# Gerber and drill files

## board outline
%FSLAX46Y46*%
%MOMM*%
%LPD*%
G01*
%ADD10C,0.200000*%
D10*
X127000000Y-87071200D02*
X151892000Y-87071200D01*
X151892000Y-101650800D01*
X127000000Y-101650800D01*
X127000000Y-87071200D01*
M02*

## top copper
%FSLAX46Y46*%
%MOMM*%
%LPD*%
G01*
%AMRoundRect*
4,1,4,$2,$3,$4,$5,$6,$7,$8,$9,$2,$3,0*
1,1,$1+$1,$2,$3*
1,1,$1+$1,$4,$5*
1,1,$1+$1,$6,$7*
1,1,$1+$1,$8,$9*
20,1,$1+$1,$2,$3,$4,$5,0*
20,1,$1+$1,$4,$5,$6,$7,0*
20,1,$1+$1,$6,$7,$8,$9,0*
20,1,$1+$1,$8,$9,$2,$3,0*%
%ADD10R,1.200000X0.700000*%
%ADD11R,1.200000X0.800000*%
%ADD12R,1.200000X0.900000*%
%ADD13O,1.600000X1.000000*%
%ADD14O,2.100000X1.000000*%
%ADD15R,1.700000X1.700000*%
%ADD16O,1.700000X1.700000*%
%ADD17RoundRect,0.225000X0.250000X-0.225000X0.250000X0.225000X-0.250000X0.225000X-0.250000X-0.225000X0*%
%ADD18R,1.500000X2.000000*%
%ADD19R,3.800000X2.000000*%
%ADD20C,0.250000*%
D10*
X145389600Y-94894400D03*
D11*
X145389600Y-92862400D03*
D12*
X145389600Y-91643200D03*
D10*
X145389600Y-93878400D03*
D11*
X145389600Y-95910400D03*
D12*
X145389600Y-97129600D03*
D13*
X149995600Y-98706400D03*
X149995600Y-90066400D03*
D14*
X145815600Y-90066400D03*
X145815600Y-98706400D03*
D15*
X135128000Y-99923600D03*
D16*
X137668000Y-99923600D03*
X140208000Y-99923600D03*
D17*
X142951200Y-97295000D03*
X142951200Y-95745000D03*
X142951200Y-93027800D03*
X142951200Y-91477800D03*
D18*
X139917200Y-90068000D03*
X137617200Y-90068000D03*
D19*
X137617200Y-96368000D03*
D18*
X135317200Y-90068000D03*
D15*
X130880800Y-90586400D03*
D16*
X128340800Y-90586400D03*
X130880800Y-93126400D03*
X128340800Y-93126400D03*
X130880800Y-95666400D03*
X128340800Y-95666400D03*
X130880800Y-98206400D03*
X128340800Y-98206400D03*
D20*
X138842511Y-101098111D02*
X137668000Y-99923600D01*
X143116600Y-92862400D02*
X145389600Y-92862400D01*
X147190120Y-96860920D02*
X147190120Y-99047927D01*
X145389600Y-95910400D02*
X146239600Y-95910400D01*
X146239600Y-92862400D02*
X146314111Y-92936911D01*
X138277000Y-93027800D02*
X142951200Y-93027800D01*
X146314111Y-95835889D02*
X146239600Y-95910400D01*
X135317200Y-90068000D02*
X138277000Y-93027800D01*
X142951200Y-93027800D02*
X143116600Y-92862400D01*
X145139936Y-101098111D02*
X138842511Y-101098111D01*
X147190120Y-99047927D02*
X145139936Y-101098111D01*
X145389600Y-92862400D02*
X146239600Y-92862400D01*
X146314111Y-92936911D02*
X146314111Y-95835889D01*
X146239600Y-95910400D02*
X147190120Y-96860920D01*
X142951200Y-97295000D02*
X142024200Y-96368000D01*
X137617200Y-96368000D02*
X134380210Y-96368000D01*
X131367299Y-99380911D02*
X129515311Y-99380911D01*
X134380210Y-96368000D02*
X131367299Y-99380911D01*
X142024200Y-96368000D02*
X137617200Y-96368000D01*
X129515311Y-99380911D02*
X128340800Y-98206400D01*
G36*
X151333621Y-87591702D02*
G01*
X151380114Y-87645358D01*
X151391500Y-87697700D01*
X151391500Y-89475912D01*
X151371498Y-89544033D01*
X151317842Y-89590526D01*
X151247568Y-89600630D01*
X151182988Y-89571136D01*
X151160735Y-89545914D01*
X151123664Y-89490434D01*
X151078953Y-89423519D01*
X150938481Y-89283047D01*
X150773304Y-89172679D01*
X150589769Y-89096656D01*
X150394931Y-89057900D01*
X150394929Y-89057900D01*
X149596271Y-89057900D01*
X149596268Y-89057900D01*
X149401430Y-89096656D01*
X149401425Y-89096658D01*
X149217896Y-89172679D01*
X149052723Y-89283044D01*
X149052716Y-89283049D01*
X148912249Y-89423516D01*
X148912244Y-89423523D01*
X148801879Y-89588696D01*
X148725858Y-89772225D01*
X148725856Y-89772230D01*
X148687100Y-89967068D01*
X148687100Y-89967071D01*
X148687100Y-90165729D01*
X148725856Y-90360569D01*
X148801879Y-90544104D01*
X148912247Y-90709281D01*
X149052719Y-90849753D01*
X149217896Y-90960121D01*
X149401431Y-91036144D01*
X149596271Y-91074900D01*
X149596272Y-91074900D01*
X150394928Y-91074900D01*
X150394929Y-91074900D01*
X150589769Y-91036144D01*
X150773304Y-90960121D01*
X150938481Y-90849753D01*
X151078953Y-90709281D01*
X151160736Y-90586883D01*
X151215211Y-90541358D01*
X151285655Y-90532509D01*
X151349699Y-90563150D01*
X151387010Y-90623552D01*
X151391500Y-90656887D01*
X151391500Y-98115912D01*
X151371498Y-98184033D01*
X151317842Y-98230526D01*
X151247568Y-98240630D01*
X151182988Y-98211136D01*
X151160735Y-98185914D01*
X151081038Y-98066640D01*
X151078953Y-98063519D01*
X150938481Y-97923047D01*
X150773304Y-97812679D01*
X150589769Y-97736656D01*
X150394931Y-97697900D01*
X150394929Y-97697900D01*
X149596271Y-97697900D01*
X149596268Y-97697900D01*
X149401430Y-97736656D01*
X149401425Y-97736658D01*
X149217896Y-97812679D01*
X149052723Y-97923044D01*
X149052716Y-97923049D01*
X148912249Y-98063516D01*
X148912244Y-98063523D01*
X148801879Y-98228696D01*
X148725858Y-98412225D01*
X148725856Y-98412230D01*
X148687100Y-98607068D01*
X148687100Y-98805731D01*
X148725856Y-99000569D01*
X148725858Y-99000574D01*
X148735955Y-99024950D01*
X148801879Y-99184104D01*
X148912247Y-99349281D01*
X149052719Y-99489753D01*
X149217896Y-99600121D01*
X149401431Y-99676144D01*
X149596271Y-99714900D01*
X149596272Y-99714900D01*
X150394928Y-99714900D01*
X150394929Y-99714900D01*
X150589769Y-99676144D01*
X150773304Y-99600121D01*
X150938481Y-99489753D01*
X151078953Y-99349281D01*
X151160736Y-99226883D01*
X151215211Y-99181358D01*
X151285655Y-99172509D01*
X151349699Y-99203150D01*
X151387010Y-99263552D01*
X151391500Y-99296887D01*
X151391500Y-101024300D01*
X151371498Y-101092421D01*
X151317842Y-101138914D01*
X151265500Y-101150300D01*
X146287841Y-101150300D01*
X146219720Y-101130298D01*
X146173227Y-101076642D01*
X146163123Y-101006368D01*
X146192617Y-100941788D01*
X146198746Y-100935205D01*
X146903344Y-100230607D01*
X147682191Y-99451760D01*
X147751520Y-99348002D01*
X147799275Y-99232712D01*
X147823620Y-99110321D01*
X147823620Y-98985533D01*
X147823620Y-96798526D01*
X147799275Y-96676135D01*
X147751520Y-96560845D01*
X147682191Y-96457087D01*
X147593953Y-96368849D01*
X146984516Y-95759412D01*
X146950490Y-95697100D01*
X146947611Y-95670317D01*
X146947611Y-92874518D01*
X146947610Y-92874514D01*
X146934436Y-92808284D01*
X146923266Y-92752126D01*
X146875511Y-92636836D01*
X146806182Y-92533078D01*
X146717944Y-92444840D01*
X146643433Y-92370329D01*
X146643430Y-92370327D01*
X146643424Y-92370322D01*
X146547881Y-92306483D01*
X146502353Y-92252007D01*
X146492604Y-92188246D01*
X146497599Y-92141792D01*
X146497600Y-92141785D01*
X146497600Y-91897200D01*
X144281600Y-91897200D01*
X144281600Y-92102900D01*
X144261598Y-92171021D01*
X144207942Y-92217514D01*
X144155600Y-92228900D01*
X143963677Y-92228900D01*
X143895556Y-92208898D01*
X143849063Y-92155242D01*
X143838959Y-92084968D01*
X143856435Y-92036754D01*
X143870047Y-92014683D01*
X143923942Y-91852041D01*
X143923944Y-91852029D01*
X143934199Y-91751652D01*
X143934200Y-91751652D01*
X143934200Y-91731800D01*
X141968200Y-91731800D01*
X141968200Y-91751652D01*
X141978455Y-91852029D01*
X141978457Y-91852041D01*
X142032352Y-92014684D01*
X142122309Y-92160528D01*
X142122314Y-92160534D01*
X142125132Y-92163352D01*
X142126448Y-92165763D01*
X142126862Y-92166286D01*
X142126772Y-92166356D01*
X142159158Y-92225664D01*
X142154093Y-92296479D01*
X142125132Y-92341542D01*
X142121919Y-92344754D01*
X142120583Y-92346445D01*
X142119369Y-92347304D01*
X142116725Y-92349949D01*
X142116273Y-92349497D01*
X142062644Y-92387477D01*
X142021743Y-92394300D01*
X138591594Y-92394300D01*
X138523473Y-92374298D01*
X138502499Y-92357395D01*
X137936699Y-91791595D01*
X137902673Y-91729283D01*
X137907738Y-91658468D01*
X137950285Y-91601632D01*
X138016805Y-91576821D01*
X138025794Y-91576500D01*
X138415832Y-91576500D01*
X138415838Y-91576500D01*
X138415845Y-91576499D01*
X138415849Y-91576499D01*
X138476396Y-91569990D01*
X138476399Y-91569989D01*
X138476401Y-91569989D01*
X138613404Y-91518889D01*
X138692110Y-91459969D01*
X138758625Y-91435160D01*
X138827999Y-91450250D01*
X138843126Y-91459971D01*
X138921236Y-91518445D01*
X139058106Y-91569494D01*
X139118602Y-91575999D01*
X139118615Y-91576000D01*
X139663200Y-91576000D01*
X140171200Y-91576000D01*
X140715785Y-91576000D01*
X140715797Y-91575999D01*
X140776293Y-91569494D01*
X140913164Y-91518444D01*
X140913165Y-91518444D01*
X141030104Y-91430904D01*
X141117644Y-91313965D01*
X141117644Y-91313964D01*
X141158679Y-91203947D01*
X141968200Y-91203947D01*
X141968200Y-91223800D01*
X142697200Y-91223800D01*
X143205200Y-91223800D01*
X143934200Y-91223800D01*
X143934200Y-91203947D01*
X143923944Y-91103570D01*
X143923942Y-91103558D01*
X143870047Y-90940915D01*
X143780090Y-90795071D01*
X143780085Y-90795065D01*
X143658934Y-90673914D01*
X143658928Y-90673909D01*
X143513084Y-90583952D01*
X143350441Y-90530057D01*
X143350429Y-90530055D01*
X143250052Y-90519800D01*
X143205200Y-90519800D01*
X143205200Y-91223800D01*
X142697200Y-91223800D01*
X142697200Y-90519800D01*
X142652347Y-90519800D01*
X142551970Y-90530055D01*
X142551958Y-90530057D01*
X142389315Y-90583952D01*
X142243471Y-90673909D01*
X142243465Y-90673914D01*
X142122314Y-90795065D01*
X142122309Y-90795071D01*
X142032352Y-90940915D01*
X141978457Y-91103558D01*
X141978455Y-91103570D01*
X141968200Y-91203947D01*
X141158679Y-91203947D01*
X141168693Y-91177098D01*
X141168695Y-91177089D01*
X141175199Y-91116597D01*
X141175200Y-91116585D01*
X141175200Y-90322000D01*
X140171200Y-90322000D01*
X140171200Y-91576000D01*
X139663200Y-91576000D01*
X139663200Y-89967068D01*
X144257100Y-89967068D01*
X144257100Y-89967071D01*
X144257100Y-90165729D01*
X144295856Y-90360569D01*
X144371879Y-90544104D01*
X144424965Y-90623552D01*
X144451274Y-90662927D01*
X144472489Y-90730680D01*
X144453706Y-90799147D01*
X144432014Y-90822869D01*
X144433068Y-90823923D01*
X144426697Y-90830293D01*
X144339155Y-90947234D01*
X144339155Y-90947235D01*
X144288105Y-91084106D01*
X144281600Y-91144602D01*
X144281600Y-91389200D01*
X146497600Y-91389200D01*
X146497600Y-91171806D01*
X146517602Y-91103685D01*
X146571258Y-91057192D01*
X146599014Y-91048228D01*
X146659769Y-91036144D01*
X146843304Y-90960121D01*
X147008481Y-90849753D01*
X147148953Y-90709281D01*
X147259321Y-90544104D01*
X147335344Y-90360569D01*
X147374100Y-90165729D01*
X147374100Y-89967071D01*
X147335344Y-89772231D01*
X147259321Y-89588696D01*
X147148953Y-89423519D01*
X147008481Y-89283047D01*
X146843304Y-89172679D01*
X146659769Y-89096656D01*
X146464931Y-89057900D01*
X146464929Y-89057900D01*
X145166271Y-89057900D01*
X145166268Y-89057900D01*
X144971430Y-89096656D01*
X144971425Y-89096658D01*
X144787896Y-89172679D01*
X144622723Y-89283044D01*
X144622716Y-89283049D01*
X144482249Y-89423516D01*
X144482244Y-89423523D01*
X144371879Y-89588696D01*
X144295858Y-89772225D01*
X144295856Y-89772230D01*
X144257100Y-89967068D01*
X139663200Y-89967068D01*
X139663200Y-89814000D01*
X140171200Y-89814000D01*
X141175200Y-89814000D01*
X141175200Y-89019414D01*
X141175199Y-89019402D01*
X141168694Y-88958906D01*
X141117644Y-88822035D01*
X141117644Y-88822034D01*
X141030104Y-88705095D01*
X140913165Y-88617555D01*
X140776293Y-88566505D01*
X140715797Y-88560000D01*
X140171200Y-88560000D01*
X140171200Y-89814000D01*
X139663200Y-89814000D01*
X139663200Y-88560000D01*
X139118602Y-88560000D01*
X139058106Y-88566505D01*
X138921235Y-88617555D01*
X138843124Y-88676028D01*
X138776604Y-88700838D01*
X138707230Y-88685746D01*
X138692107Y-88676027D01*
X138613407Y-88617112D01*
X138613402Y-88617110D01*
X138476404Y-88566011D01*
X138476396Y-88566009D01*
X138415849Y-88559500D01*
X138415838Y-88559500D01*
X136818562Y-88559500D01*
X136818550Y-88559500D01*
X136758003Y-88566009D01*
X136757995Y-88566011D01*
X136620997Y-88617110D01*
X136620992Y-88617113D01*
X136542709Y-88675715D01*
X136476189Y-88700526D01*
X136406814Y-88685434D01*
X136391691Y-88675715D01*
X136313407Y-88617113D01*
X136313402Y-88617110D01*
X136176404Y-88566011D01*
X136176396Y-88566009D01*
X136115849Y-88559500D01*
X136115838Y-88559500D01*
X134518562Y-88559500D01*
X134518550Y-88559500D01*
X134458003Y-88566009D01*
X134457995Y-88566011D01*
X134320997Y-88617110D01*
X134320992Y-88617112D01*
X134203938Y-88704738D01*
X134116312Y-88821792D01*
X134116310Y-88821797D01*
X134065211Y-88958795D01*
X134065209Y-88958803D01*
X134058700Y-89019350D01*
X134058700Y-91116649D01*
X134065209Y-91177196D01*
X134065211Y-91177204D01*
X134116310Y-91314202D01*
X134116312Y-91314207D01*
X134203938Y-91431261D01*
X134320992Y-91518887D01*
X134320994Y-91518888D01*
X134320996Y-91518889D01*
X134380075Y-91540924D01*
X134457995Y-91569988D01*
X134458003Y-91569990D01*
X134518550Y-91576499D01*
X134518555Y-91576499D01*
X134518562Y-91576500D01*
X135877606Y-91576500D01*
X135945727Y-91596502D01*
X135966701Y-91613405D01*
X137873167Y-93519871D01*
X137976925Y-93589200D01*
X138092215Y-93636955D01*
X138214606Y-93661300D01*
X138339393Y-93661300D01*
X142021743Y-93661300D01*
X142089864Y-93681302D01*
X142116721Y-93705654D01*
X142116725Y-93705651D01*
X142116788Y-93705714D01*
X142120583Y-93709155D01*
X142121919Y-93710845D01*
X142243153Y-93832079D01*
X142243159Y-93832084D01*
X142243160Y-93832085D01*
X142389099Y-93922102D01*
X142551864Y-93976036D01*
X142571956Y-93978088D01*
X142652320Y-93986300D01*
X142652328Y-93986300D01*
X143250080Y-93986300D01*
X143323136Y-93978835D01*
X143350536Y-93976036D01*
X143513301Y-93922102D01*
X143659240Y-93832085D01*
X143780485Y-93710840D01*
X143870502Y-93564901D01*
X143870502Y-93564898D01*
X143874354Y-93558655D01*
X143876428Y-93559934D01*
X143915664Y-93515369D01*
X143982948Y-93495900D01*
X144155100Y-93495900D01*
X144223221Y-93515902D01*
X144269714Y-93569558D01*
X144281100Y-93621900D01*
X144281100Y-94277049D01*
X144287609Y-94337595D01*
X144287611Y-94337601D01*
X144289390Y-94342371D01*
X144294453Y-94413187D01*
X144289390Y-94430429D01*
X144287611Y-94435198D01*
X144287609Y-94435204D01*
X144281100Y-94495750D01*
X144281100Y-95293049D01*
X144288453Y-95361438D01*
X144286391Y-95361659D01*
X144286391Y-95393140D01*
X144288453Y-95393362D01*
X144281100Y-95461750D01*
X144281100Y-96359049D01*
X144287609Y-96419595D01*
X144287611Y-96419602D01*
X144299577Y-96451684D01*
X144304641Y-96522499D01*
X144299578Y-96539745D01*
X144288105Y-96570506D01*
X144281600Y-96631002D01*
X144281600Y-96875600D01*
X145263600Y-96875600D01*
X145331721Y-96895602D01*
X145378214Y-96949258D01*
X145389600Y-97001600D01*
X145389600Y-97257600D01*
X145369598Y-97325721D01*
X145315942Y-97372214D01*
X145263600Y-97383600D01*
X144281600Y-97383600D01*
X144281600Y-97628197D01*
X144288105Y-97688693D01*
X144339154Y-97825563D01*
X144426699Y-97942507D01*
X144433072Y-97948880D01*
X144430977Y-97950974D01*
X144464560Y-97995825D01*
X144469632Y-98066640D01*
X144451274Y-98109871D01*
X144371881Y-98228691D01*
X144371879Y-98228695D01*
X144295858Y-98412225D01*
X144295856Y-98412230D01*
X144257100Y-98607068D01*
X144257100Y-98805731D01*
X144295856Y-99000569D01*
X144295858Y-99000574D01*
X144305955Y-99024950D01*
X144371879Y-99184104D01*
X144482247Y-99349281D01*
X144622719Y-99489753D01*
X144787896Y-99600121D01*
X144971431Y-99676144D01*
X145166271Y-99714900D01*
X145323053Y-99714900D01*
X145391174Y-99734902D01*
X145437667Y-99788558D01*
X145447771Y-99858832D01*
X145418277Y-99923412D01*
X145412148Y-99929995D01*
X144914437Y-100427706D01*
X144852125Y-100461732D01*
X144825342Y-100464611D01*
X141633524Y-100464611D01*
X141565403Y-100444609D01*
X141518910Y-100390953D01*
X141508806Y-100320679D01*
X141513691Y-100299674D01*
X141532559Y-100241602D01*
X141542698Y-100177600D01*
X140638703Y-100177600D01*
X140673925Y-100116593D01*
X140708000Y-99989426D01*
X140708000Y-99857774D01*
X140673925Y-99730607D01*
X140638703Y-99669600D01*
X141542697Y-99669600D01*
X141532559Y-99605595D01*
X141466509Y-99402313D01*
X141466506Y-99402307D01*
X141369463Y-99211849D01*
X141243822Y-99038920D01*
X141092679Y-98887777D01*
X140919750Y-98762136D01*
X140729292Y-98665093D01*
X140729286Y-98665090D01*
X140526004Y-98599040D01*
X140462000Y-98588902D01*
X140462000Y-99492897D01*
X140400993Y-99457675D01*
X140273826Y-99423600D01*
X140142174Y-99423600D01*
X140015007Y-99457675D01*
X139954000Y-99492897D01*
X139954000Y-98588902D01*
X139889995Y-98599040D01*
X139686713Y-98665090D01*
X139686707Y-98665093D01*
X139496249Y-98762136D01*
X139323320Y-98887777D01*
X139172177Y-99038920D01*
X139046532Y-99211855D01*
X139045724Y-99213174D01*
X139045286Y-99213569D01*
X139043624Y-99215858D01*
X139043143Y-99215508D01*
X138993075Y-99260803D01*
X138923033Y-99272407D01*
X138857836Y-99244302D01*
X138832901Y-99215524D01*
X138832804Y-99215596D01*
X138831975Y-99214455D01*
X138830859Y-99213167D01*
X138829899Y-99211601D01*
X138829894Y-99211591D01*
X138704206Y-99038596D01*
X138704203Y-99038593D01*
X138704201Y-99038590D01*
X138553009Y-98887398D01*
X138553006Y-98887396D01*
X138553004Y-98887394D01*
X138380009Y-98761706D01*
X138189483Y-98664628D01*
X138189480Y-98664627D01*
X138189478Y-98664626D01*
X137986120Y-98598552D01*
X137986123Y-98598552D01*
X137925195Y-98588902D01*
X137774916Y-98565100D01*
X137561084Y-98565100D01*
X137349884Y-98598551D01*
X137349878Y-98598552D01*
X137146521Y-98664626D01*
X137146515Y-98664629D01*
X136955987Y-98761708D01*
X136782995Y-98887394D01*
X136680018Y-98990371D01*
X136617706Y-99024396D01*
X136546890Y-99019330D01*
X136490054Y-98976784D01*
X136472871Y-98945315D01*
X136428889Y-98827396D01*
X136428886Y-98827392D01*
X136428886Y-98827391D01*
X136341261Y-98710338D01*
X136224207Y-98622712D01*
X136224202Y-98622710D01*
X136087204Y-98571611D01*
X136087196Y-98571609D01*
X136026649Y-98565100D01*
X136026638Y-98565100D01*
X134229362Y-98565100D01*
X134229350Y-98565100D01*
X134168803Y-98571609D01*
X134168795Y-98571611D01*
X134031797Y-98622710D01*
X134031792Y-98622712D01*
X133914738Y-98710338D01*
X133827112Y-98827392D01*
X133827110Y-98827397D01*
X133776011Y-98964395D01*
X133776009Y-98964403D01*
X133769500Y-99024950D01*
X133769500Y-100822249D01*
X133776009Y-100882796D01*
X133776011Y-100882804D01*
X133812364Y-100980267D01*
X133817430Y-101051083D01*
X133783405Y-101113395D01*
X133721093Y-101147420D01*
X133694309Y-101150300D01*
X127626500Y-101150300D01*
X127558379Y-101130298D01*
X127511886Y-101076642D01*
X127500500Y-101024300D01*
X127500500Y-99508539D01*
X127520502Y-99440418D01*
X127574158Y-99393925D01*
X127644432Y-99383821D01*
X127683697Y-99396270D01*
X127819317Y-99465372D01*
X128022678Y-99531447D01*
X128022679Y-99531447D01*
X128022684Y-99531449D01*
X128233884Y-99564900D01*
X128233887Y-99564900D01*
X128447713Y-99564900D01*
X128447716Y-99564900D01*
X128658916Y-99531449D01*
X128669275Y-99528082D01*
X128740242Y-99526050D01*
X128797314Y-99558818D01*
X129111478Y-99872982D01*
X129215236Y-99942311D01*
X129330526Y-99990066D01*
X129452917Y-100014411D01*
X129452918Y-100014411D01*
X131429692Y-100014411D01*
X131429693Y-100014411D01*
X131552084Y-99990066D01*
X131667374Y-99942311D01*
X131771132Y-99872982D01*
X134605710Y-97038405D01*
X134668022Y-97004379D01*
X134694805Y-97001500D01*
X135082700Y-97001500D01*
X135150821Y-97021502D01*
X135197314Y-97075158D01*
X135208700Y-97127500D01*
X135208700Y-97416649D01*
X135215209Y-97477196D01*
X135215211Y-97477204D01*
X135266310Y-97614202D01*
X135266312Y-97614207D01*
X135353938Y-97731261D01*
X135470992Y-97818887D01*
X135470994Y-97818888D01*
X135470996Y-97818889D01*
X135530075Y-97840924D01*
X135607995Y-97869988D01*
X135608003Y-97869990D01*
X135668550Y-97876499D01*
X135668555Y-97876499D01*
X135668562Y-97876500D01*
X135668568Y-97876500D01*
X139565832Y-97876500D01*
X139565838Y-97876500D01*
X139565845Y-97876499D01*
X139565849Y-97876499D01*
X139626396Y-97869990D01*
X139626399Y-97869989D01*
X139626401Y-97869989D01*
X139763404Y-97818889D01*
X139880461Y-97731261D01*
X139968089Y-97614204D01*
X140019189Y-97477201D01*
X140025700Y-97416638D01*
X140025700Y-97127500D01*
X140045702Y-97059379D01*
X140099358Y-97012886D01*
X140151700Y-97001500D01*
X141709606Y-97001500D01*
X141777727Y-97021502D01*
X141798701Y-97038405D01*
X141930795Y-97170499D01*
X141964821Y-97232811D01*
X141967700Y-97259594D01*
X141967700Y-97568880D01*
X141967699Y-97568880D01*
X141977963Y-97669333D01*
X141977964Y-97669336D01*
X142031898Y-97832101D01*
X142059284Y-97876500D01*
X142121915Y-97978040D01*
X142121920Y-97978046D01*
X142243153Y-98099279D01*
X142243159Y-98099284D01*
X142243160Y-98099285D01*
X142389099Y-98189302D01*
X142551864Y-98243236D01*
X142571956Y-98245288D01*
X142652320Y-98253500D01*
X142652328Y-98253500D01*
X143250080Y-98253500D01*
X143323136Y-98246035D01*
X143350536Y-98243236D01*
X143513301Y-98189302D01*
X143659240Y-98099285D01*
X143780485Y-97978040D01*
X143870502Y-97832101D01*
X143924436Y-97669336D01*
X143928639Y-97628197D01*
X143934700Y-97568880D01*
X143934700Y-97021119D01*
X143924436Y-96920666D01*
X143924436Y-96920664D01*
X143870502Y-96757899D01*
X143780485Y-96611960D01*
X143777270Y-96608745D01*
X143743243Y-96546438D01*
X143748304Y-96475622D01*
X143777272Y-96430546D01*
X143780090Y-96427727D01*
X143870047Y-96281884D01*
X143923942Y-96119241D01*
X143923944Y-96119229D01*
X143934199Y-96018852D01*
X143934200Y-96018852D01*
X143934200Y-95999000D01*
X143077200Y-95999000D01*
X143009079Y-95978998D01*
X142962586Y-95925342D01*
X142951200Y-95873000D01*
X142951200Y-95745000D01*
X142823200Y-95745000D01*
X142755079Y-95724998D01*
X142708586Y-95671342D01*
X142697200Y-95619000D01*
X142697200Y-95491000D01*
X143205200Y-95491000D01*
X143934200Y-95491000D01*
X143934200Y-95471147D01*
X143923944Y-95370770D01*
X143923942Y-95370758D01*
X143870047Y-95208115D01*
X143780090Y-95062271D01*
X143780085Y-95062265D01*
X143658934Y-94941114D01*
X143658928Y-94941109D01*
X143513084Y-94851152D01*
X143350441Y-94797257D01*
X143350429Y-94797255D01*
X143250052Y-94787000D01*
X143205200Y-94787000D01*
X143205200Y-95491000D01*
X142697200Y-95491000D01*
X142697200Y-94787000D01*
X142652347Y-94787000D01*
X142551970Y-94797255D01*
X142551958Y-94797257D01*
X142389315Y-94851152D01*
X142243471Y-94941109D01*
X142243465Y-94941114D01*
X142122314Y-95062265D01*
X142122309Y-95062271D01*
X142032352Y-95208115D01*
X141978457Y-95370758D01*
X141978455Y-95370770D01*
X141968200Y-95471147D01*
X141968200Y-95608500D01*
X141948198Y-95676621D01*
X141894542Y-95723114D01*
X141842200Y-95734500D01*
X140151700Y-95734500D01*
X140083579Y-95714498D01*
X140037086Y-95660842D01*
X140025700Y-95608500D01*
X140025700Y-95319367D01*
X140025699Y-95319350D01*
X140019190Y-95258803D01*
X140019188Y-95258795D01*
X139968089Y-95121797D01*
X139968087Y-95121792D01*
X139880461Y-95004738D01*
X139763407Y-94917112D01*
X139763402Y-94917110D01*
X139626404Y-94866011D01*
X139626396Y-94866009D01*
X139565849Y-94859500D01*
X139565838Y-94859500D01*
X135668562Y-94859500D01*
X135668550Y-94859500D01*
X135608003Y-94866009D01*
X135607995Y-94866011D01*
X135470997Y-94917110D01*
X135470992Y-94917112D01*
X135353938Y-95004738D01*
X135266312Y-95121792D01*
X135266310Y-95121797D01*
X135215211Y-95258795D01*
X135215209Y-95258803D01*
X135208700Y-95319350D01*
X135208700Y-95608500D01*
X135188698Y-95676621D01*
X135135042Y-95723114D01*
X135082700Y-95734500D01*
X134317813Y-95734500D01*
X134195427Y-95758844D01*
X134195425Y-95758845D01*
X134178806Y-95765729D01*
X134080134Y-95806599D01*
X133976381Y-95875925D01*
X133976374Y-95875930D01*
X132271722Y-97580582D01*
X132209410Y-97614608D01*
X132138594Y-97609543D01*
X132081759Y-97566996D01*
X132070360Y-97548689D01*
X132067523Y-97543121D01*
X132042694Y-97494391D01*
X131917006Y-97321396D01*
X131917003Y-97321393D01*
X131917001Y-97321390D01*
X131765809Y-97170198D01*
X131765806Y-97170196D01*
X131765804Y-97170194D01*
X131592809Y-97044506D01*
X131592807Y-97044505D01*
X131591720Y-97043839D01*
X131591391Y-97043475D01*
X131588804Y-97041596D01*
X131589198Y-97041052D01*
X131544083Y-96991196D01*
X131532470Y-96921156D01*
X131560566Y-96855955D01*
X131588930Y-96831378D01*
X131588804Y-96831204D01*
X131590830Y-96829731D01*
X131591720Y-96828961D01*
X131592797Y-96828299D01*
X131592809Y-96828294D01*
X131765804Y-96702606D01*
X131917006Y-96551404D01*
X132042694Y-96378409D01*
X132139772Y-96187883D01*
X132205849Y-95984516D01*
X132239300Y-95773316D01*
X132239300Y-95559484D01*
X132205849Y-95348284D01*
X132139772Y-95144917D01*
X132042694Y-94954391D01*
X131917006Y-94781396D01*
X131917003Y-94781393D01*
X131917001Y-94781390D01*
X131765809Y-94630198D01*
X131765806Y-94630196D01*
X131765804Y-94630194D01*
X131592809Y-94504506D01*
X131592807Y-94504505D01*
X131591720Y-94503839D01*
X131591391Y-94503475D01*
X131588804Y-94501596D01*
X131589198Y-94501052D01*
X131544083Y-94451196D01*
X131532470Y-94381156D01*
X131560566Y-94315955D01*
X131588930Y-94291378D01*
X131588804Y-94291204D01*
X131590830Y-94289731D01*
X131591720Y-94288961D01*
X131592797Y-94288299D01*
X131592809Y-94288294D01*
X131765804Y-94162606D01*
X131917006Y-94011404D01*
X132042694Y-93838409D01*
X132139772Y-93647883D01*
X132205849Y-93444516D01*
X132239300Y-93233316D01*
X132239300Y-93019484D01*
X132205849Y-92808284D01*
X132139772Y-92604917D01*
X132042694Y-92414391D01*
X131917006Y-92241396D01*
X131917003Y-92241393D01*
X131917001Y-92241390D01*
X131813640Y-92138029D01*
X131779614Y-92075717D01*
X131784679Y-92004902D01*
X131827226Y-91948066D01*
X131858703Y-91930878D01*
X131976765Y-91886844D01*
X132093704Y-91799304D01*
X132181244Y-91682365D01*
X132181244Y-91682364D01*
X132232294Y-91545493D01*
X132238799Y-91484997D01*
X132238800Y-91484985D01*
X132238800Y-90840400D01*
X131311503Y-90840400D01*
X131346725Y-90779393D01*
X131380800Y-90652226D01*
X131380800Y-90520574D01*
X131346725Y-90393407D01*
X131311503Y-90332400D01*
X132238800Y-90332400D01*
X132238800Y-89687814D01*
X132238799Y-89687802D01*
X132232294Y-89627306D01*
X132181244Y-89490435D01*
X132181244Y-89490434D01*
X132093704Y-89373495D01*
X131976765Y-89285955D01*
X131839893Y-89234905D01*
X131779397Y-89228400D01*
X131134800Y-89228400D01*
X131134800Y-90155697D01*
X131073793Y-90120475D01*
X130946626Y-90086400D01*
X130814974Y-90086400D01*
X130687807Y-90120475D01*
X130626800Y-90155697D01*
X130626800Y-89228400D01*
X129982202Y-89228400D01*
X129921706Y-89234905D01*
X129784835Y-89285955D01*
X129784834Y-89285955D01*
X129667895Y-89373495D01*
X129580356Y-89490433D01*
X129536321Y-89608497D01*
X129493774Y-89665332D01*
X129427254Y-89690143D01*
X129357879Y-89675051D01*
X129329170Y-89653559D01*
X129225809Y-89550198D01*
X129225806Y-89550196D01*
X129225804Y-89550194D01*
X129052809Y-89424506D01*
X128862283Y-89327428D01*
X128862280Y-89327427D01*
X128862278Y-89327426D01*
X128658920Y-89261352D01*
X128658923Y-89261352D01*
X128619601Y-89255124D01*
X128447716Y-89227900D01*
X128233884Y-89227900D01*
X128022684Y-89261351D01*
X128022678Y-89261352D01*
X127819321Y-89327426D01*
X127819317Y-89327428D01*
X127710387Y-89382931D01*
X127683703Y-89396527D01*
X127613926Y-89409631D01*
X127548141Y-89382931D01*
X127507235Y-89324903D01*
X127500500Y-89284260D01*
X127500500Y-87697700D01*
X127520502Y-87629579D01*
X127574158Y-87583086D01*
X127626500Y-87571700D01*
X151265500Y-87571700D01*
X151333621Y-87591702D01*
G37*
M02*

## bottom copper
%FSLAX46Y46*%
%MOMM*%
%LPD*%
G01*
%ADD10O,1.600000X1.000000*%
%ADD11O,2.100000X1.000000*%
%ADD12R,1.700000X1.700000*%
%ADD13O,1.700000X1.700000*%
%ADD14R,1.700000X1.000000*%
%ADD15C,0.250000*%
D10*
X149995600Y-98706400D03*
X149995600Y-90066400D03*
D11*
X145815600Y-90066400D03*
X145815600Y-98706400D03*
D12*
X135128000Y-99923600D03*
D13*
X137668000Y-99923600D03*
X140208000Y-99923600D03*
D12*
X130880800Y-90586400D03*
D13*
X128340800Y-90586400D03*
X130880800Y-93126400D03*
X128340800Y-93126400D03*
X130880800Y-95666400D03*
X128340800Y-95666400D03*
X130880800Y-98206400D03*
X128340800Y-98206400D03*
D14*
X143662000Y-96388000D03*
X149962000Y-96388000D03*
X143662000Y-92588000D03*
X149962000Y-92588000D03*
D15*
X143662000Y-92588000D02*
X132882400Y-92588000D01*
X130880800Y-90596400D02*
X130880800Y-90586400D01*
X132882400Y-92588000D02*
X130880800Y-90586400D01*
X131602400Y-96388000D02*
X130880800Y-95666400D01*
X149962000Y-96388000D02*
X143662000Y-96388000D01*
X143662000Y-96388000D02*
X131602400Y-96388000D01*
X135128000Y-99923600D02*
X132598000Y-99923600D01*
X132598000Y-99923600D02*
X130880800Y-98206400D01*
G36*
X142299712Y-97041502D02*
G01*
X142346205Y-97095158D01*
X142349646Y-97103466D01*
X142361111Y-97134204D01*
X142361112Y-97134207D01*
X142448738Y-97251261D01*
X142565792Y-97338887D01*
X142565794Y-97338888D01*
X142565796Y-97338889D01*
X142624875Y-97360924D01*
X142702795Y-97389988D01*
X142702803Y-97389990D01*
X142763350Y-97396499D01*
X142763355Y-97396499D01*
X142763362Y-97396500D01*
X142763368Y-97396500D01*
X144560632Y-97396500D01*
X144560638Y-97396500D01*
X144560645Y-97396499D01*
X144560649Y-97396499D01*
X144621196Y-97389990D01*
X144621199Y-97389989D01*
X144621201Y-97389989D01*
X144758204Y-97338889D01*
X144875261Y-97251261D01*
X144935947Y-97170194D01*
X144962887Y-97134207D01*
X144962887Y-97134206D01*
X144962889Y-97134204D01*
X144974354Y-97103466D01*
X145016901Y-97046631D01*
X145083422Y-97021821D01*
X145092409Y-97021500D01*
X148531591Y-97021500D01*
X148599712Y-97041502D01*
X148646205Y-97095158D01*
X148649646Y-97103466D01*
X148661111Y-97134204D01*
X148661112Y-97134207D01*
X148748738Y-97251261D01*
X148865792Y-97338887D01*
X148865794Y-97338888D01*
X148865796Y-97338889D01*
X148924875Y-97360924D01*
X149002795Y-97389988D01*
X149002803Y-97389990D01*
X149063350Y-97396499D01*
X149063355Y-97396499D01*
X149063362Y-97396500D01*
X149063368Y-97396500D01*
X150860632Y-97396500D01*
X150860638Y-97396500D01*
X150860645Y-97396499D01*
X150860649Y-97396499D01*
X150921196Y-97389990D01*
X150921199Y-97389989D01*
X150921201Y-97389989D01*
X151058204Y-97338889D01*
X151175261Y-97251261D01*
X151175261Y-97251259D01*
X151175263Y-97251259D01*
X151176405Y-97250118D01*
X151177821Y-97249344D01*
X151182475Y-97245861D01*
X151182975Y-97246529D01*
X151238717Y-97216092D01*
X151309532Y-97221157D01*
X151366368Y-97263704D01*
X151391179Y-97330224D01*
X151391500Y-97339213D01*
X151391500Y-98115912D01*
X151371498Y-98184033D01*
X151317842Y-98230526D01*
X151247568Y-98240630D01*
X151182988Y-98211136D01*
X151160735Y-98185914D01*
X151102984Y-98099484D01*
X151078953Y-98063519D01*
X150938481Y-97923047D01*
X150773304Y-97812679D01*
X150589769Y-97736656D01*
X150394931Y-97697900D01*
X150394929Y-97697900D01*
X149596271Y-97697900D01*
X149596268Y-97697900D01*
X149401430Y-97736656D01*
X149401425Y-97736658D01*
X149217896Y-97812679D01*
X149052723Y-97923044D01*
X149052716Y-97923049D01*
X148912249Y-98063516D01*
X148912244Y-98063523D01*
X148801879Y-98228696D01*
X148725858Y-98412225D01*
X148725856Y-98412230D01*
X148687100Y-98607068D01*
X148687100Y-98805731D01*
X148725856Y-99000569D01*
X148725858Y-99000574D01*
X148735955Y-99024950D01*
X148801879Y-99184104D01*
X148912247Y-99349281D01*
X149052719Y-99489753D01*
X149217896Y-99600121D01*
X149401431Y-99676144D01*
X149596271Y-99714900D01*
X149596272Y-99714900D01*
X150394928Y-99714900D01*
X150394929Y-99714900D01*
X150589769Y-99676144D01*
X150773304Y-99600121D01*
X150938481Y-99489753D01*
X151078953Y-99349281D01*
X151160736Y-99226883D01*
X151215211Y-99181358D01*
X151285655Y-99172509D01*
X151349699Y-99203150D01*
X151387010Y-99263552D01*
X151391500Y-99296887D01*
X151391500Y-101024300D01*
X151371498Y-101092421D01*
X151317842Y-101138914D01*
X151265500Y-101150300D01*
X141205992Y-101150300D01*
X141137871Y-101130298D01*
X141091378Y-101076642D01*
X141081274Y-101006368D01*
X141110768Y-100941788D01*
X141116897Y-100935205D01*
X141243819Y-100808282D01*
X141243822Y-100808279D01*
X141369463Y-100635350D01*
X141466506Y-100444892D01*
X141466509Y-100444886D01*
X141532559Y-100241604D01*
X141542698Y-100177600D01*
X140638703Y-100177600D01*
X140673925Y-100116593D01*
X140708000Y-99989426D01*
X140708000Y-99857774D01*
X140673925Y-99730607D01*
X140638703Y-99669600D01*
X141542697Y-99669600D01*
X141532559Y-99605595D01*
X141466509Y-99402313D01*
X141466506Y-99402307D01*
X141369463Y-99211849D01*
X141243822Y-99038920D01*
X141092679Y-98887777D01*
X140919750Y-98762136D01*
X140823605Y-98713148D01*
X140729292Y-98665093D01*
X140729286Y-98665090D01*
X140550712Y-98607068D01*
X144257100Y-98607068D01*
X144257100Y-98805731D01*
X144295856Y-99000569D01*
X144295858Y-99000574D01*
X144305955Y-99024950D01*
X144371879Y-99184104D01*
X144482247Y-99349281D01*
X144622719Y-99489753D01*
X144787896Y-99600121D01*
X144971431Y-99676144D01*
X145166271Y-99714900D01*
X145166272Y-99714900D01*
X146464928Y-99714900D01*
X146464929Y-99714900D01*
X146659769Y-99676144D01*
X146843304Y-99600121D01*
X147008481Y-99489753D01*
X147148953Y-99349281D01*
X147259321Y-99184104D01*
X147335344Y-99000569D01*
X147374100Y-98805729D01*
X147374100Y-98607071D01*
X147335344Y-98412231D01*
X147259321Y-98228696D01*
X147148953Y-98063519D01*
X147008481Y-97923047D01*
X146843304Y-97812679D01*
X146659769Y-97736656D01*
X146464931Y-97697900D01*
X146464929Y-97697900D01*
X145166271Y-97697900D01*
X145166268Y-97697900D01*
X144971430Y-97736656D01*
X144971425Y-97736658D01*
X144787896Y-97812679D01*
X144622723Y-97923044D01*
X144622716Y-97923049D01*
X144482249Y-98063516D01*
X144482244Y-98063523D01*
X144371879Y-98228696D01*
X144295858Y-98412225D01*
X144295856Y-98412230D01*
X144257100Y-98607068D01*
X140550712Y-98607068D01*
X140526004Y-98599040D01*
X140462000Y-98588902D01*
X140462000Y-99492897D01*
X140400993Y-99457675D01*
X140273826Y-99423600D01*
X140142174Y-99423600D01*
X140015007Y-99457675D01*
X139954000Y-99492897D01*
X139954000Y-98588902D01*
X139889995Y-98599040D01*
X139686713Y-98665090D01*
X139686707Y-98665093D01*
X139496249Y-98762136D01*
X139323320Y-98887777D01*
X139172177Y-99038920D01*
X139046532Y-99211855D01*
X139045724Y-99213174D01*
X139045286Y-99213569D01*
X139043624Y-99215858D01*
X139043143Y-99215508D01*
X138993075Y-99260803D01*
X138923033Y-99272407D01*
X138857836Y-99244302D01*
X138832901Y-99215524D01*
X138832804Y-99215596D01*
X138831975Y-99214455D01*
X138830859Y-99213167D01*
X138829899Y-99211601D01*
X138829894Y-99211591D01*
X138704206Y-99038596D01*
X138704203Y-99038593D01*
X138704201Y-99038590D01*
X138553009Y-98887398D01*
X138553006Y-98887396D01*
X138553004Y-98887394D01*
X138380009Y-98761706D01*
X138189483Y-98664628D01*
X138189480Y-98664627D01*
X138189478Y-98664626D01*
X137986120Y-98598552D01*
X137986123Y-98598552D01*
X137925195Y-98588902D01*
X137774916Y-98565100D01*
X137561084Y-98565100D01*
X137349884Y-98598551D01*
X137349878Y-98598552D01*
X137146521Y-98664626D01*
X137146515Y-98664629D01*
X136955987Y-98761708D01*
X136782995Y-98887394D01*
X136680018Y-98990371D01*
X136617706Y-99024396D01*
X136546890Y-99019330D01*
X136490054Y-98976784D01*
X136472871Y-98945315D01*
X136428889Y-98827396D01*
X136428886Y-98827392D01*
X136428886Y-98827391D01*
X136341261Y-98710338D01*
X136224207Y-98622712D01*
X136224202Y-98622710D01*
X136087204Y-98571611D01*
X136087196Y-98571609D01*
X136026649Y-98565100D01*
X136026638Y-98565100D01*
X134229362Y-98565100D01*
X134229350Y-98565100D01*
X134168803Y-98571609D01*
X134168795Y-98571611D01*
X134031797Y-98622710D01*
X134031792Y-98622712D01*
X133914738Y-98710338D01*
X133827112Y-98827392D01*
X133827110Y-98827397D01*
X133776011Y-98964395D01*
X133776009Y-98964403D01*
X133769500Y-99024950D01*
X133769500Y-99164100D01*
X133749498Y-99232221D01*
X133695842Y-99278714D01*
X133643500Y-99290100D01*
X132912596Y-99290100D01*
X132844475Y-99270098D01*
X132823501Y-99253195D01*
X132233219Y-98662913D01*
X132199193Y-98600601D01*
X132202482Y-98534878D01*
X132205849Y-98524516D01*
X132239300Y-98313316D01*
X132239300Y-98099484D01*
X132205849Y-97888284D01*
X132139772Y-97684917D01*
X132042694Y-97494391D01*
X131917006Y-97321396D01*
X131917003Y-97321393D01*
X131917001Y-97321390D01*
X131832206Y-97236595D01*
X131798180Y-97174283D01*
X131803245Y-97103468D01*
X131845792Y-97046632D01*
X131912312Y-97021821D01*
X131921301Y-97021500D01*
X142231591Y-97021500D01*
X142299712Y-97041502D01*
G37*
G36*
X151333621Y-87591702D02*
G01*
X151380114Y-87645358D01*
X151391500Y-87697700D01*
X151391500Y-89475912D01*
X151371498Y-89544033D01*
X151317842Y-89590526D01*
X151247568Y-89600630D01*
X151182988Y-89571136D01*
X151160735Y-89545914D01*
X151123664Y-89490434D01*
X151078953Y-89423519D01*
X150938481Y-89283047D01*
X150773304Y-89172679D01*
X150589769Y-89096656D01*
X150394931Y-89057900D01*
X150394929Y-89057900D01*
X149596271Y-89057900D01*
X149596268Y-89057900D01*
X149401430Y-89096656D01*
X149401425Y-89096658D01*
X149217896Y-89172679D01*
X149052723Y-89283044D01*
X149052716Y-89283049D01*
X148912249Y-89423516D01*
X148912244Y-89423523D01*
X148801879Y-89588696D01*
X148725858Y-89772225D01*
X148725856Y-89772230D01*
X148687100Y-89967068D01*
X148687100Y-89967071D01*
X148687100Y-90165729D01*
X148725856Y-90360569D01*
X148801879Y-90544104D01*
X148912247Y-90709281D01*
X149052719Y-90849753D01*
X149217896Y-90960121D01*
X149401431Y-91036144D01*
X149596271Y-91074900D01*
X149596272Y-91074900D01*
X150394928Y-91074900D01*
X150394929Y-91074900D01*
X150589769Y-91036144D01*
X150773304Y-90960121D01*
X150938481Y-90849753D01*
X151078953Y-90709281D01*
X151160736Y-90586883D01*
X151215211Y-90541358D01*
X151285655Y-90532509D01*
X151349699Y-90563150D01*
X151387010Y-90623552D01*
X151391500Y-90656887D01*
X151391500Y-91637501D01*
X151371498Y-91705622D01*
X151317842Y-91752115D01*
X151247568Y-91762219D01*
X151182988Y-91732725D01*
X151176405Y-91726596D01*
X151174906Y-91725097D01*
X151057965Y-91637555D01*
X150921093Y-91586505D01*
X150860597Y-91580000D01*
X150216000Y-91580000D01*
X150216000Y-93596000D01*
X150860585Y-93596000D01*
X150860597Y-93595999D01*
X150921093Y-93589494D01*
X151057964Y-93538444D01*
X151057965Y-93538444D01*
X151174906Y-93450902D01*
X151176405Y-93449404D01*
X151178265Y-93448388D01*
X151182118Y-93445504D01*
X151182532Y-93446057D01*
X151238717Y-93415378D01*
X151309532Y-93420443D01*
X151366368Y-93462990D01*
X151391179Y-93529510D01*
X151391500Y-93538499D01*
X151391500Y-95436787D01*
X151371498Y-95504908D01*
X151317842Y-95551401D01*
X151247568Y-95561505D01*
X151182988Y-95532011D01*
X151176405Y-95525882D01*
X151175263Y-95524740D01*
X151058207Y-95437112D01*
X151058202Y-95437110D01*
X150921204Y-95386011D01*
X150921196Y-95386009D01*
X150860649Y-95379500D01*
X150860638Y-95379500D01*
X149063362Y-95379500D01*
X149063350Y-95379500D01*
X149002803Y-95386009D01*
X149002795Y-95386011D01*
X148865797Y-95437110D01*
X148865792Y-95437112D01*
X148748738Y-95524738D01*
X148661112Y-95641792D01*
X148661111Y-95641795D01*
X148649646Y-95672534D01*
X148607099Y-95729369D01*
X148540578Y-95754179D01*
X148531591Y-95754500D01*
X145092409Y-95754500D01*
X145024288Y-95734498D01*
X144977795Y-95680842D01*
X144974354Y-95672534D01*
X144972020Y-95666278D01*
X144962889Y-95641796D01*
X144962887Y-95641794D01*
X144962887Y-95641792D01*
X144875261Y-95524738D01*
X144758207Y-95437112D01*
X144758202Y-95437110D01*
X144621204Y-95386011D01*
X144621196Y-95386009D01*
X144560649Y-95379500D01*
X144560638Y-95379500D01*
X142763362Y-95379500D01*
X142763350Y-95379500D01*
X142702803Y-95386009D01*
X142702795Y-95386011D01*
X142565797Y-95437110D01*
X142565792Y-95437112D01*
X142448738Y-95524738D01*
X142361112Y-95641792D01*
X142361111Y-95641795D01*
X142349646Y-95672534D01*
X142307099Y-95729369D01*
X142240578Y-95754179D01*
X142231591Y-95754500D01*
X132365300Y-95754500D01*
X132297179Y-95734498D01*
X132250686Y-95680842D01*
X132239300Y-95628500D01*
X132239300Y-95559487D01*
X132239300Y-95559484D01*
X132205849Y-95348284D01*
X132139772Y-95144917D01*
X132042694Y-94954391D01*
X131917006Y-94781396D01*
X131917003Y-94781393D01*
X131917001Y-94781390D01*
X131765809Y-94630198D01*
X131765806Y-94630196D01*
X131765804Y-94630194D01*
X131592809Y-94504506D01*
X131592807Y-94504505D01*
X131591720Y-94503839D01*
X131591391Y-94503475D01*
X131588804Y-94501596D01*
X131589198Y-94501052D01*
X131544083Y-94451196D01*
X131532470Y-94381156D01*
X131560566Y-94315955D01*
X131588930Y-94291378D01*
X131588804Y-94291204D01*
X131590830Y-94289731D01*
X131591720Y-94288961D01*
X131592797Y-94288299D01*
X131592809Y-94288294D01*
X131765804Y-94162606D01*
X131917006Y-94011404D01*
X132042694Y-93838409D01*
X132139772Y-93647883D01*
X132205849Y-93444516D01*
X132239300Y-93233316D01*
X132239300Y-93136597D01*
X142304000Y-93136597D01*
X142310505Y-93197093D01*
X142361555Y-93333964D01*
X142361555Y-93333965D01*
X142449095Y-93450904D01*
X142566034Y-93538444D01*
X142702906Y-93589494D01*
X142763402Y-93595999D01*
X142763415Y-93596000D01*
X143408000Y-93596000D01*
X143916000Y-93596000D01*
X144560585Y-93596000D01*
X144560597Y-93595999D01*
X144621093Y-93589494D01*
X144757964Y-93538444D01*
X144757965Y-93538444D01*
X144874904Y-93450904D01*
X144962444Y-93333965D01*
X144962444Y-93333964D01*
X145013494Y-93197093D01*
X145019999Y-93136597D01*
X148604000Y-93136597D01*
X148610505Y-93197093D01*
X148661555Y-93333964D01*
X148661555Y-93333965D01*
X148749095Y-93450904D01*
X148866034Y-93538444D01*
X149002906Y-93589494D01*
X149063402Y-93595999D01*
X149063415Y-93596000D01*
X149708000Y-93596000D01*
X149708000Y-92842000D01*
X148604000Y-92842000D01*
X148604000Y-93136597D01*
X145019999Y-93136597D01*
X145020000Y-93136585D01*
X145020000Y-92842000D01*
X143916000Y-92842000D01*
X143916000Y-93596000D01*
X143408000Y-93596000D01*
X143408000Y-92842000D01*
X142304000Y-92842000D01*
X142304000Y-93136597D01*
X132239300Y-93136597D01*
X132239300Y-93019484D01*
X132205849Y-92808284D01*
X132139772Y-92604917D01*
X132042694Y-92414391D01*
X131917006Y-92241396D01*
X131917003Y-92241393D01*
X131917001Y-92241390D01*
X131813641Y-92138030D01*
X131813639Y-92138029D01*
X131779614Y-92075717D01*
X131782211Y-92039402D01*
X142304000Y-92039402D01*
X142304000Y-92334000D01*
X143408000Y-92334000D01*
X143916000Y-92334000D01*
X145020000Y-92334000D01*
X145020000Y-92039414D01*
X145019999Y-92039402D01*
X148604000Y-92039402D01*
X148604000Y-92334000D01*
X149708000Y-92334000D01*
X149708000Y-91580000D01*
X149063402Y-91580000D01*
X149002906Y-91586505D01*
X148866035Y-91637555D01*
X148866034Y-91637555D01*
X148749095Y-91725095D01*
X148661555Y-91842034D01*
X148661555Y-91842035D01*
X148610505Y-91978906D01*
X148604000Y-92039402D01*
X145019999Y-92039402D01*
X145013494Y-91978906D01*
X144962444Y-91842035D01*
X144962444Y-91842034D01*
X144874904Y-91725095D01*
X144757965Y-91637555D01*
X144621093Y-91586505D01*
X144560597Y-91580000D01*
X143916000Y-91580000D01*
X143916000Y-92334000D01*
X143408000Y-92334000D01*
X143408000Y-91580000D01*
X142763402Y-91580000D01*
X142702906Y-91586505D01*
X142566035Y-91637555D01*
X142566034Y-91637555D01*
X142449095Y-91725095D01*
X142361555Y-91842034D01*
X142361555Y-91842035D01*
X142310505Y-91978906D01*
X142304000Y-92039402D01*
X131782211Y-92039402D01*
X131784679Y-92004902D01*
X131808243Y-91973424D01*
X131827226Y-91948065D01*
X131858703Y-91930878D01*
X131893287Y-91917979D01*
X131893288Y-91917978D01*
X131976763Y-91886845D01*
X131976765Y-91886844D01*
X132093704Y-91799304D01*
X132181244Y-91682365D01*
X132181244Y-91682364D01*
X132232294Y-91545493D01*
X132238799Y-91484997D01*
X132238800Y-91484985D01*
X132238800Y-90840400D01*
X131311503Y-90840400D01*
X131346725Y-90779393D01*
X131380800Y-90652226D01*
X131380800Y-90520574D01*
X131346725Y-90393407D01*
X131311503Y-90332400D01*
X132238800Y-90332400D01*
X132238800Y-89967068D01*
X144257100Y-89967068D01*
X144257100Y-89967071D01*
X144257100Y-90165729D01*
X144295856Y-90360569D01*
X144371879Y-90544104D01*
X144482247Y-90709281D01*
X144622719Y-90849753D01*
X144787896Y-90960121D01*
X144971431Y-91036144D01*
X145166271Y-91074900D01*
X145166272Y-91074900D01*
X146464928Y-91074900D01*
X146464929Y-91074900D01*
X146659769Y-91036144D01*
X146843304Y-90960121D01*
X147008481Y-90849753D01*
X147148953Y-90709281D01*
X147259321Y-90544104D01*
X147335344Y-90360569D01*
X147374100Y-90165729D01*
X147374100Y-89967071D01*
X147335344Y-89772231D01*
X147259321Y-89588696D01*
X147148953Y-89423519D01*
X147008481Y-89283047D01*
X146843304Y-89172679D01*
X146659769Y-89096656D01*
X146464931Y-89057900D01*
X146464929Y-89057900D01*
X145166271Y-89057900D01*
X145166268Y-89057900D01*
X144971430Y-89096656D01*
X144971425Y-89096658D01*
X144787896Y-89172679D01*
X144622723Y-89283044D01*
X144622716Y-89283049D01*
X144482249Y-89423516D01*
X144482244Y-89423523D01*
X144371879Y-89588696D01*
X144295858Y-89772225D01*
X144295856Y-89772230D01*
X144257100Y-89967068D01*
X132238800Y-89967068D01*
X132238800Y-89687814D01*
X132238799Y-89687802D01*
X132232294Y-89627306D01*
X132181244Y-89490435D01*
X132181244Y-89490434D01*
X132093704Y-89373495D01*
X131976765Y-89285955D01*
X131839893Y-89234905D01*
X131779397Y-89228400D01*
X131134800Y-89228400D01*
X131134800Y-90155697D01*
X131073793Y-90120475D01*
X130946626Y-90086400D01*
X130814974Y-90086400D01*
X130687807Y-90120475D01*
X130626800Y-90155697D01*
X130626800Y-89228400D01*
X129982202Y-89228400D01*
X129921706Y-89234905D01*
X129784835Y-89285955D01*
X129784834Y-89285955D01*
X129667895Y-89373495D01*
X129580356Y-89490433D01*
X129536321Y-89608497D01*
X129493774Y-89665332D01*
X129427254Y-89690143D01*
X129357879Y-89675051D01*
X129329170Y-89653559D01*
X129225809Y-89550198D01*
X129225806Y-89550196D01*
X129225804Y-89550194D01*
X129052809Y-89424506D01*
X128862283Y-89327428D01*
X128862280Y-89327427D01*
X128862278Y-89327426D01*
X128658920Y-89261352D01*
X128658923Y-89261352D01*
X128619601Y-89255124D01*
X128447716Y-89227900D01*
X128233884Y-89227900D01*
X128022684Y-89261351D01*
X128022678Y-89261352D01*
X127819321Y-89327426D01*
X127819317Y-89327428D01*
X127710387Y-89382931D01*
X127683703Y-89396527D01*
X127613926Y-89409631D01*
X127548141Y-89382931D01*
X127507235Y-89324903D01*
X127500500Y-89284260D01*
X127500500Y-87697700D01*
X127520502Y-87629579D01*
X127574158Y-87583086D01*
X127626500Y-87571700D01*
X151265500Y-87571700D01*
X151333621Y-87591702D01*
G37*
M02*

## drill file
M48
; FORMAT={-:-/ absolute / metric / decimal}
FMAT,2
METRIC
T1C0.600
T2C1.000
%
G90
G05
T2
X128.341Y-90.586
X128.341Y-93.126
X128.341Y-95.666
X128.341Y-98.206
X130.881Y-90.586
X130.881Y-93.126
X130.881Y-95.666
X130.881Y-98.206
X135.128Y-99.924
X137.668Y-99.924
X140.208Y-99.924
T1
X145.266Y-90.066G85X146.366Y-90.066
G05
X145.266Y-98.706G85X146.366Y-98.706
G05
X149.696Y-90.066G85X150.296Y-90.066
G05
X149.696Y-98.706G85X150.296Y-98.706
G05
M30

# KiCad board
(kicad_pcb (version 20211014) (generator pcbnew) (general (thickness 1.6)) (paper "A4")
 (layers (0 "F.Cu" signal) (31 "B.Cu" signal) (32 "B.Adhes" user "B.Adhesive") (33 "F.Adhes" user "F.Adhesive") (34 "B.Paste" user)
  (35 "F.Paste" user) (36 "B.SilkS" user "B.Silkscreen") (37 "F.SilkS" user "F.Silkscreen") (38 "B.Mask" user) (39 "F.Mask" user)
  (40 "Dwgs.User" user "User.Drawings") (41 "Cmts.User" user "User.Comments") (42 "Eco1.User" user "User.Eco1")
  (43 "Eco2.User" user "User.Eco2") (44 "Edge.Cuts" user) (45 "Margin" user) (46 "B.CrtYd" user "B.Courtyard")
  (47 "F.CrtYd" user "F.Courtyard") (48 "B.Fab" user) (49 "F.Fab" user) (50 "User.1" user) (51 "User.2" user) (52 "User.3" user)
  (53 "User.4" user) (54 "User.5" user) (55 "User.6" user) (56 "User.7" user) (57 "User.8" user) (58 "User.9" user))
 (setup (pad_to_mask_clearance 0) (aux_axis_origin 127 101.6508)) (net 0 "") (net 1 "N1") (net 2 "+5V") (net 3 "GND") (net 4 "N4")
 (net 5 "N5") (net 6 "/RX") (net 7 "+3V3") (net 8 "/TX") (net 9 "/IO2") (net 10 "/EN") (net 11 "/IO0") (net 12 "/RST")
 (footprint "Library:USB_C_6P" (layer "F.Cu") (at 148.9456 94.3864 90)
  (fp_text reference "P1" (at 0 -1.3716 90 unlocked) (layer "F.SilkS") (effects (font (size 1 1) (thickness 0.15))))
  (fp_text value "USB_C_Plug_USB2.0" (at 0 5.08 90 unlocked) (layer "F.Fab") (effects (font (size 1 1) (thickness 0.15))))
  (pad "A5" smd rect (at -0.508 -3.556 90) (size 0.7 1.2) (layers "F.Cu" "F.Paste" "F.Mask") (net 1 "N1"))
  (pad "A9" smd rect (at 1.524 -3.556 90) (size 0.8 1.2) (layers "F.Cu" "F.Paste" "F.Mask") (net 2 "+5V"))
  (pad "A12" smd rect (at 2.7432 -3.556 90) (size 0.9 1.2) (layers "F.Cu" "F.Paste" "F.Mask") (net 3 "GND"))
  (pad "B5" smd rect (at 0.508 -3.556 90) (size 0.7 1.2) (layers "F.Cu" "F.Paste" "F.Mask") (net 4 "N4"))
  (pad "B9" smd rect (at -1.524 -3.556 90) (size 0.8 1.2) (layers "F.Cu" "F.Paste" "F.Mask") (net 2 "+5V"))
  (pad "B12" smd rect (at -2.7432 -3.556 90) (size 0.9 1.2) (layers "F.Cu" "F.Paste" "F.Mask") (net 3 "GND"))
  (pad "S1" thru_hole oval (at -4.32 1.05 90) (size 1 1.6) (drill oval 0.6 1.2) (layers *.Cu *.Mask) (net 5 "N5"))
  (pad "S1" thru_hole oval (at 4.32 1.05 90) (size 1 1.6) (drill oval 0.6 1.2) (layers *.Cu *.Mask) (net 5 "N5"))
  (pad "S1" thru_hole oval (at 4.32 -3.13 90) (size 1 2.1) (drill oval 0.6 1.7) (layers *.Cu *.Mask) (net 5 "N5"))
  (pad "S1" thru_hole oval (at -4.32 -3.13 90) (size 1 2.1) (drill oval 0.6 1.7) (layers *.Cu *.Mask) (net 5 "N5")))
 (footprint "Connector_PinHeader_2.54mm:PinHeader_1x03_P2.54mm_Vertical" (layer "F.Cu") (at 135.128 99.9236 90)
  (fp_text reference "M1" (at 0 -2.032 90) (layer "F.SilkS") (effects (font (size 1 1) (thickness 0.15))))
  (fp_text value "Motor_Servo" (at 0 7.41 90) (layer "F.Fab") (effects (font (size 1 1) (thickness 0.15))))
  (pad "1" thru_hole rect (at 0 0 90) (size 1.7 1.7) (drill 1) (layers *.Cu *.Mask) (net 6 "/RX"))
  (pad "2" thru_hole oval (at 0 2.54 90) (size 1.7 1.7) (drill 1) (layers *.Cu *.Mask) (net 2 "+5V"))
  (pad "3" thru_hole oval (at 0 5.08 90) (size 1.7 1.7) (drill 1) (layers *.Cu *.Mask) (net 3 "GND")))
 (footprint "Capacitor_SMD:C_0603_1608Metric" (layer "F.Cu") (at 142.9512 96.52 90)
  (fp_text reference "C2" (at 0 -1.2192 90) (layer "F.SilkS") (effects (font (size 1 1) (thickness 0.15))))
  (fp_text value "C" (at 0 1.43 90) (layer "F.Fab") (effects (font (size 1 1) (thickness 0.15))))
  (pad "1" smd roundrect (at -0.775 0 90) (size 0.9 0.95) (layers "F.Cu" "F.Paste" "F.Mask") (roundrect_rratio 0.25) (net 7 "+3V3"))
  (pad "2" smd roundrect (at 0.775 0 90) (size 0.9 0.95) (layers "F.Cu" "F.Paste" "F.Mask") (roundrect_rratio 0.25) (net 3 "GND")))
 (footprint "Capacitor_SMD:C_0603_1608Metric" (layer "F.Cu") (at 142.9512 92.2528 90)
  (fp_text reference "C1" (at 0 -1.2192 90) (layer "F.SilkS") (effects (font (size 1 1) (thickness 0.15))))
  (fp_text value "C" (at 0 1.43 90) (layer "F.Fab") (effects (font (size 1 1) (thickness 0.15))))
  (pad "1" smd roundrect (at -0.775 0 90) (size 0.9 0.95) (layers "F.Cu" "F.Paste" "F.Mask") (roundrect_rratio 0.25) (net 2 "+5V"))
  (pad "2" smd roundrect (at 0.775 0 90) (size 0.9 0.95) (layers "F.Cu" "F.Paste" "F.Mask") (roundrect_rratio 0.25) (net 3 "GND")))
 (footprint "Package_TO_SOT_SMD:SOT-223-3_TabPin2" (layer "F.Cu") (at 137.6172 93.218 -90)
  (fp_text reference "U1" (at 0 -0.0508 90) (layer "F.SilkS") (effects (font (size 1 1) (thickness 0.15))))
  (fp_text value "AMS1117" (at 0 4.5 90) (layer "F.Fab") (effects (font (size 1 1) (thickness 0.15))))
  (pad "1" smd rect (at -3.15 -2.3 270) (size 2 1.5) (layers "F.Cu" "F.Paste" "F.Mask") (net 3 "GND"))
  (pad "2" smd rect (at -3.15 0 270) (size 2 1.5) (layers "F.Cu" "F.Paste" "F.Mask") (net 7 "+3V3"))
  (pad "2" smd rect (at 3.15 0 270) (size 2 3.8) (layers "F.Cu" "F.Paste" "F.Mask") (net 7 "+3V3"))
  (pad "3" smd rect (at -3.15 2.3 270) (size 2 1.5) (layers "F.Cu" "F.Paste" "F.Mask") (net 2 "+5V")))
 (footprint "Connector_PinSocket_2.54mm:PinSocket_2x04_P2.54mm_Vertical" (layer "F.Cu") (at 130.8808 90.5864)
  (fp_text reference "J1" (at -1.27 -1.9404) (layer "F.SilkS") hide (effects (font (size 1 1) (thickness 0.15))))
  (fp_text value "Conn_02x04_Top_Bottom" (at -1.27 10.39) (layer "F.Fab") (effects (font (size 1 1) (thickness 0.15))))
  (pad "1" thru_hole rect (at 0 0) (size 1.7 1.7) (drill 1) (layers *.Cu *.Mask) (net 3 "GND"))
  (pad "2" thru_hole oval (at -2.54 0) (size 1.7 1.7) (drill 1) (layers *.Cu *.Mask) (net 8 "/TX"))
  (pad "3" thru_hole oval (at 0 2.54) (size 1.7 1.7) (drill 1) (layers *.Cu *.Mask) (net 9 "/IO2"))
  (pad "4" thru_hole oval (at -2.54 2.54) (size 1.7 1.7) (drill 1) (layers *.Cu *.Mask) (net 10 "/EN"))
  (pad "5" thru_hole oval (at 0 5.08) (size 1.7 1.7) (drill 1) (layers *.Cu *.Mask) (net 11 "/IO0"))
  (pad "6" thru_hole oval (at -2.54 5.08) (size 1.7 1.7) (drill 1) (layers *.Cu *.Mask) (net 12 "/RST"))
  (pad "7" thru_hole oval (at 0 7.62) (size 1.7 1.7) (drill 1) (layers *.Cu *.Mask) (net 6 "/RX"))
  (pad "8" thru_hole oval (at -2.54 7.62) (size 1.7 1.7) (drill 1) (layers *.Cu *.Mask) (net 7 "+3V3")))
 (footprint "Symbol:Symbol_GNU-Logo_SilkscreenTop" (layer "B.Cu") (at 137.92581 91.89593 180)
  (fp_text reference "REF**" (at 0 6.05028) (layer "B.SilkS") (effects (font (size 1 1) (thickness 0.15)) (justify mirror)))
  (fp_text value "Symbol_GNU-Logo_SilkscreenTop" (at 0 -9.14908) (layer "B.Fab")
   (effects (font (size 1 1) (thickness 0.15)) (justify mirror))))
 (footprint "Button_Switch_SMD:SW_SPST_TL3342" (layer "B.Cu") (at 146.812 94.488)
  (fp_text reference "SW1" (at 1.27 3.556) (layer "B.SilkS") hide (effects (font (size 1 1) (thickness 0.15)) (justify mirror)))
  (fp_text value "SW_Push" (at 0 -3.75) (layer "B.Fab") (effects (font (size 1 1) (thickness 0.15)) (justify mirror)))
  (pad "1" smd rect (at -3.15 1.9) (size 1.7 1) (layers "B.Cu" "B.Paste" "B.Mask") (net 11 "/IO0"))
  (pad "1" smd rect (at 3.15 1.9) (size 1.7 1) (layers "B.Cu" "B.Paste" "B.Mask") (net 11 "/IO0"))
  (pad "2" smd rect (at -3.15 -1.9) (size 1.7 1) (layers "B.Cu" "B.Paste" "B.Mask") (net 3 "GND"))
  (pad "2" smd rect (at 3.15 -1.9) (size 1.7 1) (layers "B.Cu" "B.Paste" "B.Mask") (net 3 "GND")))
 (gr_rect (start 127 101.6508) (end 151.892 87.0712) (layer "Edge.Cuts") (width 0.2) (fill none))
 (segment (start 138.842511 101.098111) (end 137.668 99.9236) (width 0.25) (layer "F.Cu") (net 2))
 (segment (start 143.1166 92.8624) (end 145.3896 92.8624) (width 0.25) (layer "F.Cu") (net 2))
 (segment (start 147.19012 96.86092) (end 147.19012 99.047927) (width 0.25) (layer "F.Cu") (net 2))
 (segment (start 145.3896 95.9104) (end 146.2396 95.9104) (width 0.25) (layer "F.Cu") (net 2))
 (segment (start 146.2396 92.8624) (end 146.314111 92.936911) (width 0.25) (layer "F.Cu") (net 2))
 (segment (start 138.277 93.0278) (end 142.9512 93.0278) (width 0.25) (layer "F.Cu") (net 2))
 (segment (start 146.314111 95.835889) (end 146.2396 95.9104) (width 0.25) (layer "F.Cu") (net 2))
 (segment (start 135.3172 90.068) (end 138.277 93.0278) (width 0.25) (layer "F.Cu") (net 2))
 (segment (start 142.9512 93.0278) (end 143.1166 92.8624) (width 0.25) (layer "F.Cu") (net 2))
 (segment (start 145.139936 101.098111) (end 138.842511 101.098111) (width 0.25) (layer "F.Cu") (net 2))
 (segment (start 147.19012 99.047927) (end 145.139936 101.098111) (width 0.25) (layer "F.Cu") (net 2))
 (segment (start 145.3896 92.8624) (end 146.2396 92.8624) (width 0.25) (layer "F.Cu") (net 2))
 (segment (start 146.314111 92.936911) (end 146.314111 95.835889) (width 0.25) (layer "F.Cu") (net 2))
 (segment (start 146.2396 95.9104) (end 147.19012 96.86092) (width 0.25) (layer "F.Cu") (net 2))
 (segment (start 143.662 92.588) (end 132.8824 92.588) (width 0.25) (layer "B.Cu") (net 3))
 (segment (start 130.8808 90.5964) (end 130.8808 90.5864) (width 0.25) (layer "B.Cu") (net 3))
 (segment (start 132.8824 92.588) (end 130.8808 90.5864) (width 0.25) (layer "B.Cu") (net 3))
 (segment (start 142.9512 97.295) (end 142.0242 96.368) (width 0.25) (layer "F.Cu") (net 7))
 (segment (start 137.6172 96.368) (end 134.38021 96.368) (width 0.25) (layer "F.Cu") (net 7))
 (segment (start 131.367299 99.380911) (end 129.515311 99.380911) (width 0.25) (layer "F.Cu") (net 7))
 (segment (start 134.38021 96.368) (end 131.367299 99.380911) (width 0.25) (layer "F.Cu") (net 7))
 (segment (start 142.0242 96.368) (end 137.6172 96.368) (width 0.25) (layer "F.Cu") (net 7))
 (segment (start 129.515311 99.380911) (end 128.3408 98.2064) (width 0.25) (layer "F.Cu") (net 7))
 (segment (start 131.6024 96.388) (end 130.8808 95.6664) (width 0.25) (layer "B.Cu") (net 11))
 (segment (start 149.962 96.388) (end 143.662 96.388) (width 0.25) (layer "B.Cu") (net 11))
 (segment (start 143.662 96.388) (end 131.6024 96.388) (width 0.25) (layer "B.Cu") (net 11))
 (segment (start 135.128 99.9236) (end 132.598 99.9236) (width 0.25) (layer "B.Cu") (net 6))
 (segment (start 132.598 99.9236) (end 130.8808 98.2064) (width 0.25) (layer "B.Cu") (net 6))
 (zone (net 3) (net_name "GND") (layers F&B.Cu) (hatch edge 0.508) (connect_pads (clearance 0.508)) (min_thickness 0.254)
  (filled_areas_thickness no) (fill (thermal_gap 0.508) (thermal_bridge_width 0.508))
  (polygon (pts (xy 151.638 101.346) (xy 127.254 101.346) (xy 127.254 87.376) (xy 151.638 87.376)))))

